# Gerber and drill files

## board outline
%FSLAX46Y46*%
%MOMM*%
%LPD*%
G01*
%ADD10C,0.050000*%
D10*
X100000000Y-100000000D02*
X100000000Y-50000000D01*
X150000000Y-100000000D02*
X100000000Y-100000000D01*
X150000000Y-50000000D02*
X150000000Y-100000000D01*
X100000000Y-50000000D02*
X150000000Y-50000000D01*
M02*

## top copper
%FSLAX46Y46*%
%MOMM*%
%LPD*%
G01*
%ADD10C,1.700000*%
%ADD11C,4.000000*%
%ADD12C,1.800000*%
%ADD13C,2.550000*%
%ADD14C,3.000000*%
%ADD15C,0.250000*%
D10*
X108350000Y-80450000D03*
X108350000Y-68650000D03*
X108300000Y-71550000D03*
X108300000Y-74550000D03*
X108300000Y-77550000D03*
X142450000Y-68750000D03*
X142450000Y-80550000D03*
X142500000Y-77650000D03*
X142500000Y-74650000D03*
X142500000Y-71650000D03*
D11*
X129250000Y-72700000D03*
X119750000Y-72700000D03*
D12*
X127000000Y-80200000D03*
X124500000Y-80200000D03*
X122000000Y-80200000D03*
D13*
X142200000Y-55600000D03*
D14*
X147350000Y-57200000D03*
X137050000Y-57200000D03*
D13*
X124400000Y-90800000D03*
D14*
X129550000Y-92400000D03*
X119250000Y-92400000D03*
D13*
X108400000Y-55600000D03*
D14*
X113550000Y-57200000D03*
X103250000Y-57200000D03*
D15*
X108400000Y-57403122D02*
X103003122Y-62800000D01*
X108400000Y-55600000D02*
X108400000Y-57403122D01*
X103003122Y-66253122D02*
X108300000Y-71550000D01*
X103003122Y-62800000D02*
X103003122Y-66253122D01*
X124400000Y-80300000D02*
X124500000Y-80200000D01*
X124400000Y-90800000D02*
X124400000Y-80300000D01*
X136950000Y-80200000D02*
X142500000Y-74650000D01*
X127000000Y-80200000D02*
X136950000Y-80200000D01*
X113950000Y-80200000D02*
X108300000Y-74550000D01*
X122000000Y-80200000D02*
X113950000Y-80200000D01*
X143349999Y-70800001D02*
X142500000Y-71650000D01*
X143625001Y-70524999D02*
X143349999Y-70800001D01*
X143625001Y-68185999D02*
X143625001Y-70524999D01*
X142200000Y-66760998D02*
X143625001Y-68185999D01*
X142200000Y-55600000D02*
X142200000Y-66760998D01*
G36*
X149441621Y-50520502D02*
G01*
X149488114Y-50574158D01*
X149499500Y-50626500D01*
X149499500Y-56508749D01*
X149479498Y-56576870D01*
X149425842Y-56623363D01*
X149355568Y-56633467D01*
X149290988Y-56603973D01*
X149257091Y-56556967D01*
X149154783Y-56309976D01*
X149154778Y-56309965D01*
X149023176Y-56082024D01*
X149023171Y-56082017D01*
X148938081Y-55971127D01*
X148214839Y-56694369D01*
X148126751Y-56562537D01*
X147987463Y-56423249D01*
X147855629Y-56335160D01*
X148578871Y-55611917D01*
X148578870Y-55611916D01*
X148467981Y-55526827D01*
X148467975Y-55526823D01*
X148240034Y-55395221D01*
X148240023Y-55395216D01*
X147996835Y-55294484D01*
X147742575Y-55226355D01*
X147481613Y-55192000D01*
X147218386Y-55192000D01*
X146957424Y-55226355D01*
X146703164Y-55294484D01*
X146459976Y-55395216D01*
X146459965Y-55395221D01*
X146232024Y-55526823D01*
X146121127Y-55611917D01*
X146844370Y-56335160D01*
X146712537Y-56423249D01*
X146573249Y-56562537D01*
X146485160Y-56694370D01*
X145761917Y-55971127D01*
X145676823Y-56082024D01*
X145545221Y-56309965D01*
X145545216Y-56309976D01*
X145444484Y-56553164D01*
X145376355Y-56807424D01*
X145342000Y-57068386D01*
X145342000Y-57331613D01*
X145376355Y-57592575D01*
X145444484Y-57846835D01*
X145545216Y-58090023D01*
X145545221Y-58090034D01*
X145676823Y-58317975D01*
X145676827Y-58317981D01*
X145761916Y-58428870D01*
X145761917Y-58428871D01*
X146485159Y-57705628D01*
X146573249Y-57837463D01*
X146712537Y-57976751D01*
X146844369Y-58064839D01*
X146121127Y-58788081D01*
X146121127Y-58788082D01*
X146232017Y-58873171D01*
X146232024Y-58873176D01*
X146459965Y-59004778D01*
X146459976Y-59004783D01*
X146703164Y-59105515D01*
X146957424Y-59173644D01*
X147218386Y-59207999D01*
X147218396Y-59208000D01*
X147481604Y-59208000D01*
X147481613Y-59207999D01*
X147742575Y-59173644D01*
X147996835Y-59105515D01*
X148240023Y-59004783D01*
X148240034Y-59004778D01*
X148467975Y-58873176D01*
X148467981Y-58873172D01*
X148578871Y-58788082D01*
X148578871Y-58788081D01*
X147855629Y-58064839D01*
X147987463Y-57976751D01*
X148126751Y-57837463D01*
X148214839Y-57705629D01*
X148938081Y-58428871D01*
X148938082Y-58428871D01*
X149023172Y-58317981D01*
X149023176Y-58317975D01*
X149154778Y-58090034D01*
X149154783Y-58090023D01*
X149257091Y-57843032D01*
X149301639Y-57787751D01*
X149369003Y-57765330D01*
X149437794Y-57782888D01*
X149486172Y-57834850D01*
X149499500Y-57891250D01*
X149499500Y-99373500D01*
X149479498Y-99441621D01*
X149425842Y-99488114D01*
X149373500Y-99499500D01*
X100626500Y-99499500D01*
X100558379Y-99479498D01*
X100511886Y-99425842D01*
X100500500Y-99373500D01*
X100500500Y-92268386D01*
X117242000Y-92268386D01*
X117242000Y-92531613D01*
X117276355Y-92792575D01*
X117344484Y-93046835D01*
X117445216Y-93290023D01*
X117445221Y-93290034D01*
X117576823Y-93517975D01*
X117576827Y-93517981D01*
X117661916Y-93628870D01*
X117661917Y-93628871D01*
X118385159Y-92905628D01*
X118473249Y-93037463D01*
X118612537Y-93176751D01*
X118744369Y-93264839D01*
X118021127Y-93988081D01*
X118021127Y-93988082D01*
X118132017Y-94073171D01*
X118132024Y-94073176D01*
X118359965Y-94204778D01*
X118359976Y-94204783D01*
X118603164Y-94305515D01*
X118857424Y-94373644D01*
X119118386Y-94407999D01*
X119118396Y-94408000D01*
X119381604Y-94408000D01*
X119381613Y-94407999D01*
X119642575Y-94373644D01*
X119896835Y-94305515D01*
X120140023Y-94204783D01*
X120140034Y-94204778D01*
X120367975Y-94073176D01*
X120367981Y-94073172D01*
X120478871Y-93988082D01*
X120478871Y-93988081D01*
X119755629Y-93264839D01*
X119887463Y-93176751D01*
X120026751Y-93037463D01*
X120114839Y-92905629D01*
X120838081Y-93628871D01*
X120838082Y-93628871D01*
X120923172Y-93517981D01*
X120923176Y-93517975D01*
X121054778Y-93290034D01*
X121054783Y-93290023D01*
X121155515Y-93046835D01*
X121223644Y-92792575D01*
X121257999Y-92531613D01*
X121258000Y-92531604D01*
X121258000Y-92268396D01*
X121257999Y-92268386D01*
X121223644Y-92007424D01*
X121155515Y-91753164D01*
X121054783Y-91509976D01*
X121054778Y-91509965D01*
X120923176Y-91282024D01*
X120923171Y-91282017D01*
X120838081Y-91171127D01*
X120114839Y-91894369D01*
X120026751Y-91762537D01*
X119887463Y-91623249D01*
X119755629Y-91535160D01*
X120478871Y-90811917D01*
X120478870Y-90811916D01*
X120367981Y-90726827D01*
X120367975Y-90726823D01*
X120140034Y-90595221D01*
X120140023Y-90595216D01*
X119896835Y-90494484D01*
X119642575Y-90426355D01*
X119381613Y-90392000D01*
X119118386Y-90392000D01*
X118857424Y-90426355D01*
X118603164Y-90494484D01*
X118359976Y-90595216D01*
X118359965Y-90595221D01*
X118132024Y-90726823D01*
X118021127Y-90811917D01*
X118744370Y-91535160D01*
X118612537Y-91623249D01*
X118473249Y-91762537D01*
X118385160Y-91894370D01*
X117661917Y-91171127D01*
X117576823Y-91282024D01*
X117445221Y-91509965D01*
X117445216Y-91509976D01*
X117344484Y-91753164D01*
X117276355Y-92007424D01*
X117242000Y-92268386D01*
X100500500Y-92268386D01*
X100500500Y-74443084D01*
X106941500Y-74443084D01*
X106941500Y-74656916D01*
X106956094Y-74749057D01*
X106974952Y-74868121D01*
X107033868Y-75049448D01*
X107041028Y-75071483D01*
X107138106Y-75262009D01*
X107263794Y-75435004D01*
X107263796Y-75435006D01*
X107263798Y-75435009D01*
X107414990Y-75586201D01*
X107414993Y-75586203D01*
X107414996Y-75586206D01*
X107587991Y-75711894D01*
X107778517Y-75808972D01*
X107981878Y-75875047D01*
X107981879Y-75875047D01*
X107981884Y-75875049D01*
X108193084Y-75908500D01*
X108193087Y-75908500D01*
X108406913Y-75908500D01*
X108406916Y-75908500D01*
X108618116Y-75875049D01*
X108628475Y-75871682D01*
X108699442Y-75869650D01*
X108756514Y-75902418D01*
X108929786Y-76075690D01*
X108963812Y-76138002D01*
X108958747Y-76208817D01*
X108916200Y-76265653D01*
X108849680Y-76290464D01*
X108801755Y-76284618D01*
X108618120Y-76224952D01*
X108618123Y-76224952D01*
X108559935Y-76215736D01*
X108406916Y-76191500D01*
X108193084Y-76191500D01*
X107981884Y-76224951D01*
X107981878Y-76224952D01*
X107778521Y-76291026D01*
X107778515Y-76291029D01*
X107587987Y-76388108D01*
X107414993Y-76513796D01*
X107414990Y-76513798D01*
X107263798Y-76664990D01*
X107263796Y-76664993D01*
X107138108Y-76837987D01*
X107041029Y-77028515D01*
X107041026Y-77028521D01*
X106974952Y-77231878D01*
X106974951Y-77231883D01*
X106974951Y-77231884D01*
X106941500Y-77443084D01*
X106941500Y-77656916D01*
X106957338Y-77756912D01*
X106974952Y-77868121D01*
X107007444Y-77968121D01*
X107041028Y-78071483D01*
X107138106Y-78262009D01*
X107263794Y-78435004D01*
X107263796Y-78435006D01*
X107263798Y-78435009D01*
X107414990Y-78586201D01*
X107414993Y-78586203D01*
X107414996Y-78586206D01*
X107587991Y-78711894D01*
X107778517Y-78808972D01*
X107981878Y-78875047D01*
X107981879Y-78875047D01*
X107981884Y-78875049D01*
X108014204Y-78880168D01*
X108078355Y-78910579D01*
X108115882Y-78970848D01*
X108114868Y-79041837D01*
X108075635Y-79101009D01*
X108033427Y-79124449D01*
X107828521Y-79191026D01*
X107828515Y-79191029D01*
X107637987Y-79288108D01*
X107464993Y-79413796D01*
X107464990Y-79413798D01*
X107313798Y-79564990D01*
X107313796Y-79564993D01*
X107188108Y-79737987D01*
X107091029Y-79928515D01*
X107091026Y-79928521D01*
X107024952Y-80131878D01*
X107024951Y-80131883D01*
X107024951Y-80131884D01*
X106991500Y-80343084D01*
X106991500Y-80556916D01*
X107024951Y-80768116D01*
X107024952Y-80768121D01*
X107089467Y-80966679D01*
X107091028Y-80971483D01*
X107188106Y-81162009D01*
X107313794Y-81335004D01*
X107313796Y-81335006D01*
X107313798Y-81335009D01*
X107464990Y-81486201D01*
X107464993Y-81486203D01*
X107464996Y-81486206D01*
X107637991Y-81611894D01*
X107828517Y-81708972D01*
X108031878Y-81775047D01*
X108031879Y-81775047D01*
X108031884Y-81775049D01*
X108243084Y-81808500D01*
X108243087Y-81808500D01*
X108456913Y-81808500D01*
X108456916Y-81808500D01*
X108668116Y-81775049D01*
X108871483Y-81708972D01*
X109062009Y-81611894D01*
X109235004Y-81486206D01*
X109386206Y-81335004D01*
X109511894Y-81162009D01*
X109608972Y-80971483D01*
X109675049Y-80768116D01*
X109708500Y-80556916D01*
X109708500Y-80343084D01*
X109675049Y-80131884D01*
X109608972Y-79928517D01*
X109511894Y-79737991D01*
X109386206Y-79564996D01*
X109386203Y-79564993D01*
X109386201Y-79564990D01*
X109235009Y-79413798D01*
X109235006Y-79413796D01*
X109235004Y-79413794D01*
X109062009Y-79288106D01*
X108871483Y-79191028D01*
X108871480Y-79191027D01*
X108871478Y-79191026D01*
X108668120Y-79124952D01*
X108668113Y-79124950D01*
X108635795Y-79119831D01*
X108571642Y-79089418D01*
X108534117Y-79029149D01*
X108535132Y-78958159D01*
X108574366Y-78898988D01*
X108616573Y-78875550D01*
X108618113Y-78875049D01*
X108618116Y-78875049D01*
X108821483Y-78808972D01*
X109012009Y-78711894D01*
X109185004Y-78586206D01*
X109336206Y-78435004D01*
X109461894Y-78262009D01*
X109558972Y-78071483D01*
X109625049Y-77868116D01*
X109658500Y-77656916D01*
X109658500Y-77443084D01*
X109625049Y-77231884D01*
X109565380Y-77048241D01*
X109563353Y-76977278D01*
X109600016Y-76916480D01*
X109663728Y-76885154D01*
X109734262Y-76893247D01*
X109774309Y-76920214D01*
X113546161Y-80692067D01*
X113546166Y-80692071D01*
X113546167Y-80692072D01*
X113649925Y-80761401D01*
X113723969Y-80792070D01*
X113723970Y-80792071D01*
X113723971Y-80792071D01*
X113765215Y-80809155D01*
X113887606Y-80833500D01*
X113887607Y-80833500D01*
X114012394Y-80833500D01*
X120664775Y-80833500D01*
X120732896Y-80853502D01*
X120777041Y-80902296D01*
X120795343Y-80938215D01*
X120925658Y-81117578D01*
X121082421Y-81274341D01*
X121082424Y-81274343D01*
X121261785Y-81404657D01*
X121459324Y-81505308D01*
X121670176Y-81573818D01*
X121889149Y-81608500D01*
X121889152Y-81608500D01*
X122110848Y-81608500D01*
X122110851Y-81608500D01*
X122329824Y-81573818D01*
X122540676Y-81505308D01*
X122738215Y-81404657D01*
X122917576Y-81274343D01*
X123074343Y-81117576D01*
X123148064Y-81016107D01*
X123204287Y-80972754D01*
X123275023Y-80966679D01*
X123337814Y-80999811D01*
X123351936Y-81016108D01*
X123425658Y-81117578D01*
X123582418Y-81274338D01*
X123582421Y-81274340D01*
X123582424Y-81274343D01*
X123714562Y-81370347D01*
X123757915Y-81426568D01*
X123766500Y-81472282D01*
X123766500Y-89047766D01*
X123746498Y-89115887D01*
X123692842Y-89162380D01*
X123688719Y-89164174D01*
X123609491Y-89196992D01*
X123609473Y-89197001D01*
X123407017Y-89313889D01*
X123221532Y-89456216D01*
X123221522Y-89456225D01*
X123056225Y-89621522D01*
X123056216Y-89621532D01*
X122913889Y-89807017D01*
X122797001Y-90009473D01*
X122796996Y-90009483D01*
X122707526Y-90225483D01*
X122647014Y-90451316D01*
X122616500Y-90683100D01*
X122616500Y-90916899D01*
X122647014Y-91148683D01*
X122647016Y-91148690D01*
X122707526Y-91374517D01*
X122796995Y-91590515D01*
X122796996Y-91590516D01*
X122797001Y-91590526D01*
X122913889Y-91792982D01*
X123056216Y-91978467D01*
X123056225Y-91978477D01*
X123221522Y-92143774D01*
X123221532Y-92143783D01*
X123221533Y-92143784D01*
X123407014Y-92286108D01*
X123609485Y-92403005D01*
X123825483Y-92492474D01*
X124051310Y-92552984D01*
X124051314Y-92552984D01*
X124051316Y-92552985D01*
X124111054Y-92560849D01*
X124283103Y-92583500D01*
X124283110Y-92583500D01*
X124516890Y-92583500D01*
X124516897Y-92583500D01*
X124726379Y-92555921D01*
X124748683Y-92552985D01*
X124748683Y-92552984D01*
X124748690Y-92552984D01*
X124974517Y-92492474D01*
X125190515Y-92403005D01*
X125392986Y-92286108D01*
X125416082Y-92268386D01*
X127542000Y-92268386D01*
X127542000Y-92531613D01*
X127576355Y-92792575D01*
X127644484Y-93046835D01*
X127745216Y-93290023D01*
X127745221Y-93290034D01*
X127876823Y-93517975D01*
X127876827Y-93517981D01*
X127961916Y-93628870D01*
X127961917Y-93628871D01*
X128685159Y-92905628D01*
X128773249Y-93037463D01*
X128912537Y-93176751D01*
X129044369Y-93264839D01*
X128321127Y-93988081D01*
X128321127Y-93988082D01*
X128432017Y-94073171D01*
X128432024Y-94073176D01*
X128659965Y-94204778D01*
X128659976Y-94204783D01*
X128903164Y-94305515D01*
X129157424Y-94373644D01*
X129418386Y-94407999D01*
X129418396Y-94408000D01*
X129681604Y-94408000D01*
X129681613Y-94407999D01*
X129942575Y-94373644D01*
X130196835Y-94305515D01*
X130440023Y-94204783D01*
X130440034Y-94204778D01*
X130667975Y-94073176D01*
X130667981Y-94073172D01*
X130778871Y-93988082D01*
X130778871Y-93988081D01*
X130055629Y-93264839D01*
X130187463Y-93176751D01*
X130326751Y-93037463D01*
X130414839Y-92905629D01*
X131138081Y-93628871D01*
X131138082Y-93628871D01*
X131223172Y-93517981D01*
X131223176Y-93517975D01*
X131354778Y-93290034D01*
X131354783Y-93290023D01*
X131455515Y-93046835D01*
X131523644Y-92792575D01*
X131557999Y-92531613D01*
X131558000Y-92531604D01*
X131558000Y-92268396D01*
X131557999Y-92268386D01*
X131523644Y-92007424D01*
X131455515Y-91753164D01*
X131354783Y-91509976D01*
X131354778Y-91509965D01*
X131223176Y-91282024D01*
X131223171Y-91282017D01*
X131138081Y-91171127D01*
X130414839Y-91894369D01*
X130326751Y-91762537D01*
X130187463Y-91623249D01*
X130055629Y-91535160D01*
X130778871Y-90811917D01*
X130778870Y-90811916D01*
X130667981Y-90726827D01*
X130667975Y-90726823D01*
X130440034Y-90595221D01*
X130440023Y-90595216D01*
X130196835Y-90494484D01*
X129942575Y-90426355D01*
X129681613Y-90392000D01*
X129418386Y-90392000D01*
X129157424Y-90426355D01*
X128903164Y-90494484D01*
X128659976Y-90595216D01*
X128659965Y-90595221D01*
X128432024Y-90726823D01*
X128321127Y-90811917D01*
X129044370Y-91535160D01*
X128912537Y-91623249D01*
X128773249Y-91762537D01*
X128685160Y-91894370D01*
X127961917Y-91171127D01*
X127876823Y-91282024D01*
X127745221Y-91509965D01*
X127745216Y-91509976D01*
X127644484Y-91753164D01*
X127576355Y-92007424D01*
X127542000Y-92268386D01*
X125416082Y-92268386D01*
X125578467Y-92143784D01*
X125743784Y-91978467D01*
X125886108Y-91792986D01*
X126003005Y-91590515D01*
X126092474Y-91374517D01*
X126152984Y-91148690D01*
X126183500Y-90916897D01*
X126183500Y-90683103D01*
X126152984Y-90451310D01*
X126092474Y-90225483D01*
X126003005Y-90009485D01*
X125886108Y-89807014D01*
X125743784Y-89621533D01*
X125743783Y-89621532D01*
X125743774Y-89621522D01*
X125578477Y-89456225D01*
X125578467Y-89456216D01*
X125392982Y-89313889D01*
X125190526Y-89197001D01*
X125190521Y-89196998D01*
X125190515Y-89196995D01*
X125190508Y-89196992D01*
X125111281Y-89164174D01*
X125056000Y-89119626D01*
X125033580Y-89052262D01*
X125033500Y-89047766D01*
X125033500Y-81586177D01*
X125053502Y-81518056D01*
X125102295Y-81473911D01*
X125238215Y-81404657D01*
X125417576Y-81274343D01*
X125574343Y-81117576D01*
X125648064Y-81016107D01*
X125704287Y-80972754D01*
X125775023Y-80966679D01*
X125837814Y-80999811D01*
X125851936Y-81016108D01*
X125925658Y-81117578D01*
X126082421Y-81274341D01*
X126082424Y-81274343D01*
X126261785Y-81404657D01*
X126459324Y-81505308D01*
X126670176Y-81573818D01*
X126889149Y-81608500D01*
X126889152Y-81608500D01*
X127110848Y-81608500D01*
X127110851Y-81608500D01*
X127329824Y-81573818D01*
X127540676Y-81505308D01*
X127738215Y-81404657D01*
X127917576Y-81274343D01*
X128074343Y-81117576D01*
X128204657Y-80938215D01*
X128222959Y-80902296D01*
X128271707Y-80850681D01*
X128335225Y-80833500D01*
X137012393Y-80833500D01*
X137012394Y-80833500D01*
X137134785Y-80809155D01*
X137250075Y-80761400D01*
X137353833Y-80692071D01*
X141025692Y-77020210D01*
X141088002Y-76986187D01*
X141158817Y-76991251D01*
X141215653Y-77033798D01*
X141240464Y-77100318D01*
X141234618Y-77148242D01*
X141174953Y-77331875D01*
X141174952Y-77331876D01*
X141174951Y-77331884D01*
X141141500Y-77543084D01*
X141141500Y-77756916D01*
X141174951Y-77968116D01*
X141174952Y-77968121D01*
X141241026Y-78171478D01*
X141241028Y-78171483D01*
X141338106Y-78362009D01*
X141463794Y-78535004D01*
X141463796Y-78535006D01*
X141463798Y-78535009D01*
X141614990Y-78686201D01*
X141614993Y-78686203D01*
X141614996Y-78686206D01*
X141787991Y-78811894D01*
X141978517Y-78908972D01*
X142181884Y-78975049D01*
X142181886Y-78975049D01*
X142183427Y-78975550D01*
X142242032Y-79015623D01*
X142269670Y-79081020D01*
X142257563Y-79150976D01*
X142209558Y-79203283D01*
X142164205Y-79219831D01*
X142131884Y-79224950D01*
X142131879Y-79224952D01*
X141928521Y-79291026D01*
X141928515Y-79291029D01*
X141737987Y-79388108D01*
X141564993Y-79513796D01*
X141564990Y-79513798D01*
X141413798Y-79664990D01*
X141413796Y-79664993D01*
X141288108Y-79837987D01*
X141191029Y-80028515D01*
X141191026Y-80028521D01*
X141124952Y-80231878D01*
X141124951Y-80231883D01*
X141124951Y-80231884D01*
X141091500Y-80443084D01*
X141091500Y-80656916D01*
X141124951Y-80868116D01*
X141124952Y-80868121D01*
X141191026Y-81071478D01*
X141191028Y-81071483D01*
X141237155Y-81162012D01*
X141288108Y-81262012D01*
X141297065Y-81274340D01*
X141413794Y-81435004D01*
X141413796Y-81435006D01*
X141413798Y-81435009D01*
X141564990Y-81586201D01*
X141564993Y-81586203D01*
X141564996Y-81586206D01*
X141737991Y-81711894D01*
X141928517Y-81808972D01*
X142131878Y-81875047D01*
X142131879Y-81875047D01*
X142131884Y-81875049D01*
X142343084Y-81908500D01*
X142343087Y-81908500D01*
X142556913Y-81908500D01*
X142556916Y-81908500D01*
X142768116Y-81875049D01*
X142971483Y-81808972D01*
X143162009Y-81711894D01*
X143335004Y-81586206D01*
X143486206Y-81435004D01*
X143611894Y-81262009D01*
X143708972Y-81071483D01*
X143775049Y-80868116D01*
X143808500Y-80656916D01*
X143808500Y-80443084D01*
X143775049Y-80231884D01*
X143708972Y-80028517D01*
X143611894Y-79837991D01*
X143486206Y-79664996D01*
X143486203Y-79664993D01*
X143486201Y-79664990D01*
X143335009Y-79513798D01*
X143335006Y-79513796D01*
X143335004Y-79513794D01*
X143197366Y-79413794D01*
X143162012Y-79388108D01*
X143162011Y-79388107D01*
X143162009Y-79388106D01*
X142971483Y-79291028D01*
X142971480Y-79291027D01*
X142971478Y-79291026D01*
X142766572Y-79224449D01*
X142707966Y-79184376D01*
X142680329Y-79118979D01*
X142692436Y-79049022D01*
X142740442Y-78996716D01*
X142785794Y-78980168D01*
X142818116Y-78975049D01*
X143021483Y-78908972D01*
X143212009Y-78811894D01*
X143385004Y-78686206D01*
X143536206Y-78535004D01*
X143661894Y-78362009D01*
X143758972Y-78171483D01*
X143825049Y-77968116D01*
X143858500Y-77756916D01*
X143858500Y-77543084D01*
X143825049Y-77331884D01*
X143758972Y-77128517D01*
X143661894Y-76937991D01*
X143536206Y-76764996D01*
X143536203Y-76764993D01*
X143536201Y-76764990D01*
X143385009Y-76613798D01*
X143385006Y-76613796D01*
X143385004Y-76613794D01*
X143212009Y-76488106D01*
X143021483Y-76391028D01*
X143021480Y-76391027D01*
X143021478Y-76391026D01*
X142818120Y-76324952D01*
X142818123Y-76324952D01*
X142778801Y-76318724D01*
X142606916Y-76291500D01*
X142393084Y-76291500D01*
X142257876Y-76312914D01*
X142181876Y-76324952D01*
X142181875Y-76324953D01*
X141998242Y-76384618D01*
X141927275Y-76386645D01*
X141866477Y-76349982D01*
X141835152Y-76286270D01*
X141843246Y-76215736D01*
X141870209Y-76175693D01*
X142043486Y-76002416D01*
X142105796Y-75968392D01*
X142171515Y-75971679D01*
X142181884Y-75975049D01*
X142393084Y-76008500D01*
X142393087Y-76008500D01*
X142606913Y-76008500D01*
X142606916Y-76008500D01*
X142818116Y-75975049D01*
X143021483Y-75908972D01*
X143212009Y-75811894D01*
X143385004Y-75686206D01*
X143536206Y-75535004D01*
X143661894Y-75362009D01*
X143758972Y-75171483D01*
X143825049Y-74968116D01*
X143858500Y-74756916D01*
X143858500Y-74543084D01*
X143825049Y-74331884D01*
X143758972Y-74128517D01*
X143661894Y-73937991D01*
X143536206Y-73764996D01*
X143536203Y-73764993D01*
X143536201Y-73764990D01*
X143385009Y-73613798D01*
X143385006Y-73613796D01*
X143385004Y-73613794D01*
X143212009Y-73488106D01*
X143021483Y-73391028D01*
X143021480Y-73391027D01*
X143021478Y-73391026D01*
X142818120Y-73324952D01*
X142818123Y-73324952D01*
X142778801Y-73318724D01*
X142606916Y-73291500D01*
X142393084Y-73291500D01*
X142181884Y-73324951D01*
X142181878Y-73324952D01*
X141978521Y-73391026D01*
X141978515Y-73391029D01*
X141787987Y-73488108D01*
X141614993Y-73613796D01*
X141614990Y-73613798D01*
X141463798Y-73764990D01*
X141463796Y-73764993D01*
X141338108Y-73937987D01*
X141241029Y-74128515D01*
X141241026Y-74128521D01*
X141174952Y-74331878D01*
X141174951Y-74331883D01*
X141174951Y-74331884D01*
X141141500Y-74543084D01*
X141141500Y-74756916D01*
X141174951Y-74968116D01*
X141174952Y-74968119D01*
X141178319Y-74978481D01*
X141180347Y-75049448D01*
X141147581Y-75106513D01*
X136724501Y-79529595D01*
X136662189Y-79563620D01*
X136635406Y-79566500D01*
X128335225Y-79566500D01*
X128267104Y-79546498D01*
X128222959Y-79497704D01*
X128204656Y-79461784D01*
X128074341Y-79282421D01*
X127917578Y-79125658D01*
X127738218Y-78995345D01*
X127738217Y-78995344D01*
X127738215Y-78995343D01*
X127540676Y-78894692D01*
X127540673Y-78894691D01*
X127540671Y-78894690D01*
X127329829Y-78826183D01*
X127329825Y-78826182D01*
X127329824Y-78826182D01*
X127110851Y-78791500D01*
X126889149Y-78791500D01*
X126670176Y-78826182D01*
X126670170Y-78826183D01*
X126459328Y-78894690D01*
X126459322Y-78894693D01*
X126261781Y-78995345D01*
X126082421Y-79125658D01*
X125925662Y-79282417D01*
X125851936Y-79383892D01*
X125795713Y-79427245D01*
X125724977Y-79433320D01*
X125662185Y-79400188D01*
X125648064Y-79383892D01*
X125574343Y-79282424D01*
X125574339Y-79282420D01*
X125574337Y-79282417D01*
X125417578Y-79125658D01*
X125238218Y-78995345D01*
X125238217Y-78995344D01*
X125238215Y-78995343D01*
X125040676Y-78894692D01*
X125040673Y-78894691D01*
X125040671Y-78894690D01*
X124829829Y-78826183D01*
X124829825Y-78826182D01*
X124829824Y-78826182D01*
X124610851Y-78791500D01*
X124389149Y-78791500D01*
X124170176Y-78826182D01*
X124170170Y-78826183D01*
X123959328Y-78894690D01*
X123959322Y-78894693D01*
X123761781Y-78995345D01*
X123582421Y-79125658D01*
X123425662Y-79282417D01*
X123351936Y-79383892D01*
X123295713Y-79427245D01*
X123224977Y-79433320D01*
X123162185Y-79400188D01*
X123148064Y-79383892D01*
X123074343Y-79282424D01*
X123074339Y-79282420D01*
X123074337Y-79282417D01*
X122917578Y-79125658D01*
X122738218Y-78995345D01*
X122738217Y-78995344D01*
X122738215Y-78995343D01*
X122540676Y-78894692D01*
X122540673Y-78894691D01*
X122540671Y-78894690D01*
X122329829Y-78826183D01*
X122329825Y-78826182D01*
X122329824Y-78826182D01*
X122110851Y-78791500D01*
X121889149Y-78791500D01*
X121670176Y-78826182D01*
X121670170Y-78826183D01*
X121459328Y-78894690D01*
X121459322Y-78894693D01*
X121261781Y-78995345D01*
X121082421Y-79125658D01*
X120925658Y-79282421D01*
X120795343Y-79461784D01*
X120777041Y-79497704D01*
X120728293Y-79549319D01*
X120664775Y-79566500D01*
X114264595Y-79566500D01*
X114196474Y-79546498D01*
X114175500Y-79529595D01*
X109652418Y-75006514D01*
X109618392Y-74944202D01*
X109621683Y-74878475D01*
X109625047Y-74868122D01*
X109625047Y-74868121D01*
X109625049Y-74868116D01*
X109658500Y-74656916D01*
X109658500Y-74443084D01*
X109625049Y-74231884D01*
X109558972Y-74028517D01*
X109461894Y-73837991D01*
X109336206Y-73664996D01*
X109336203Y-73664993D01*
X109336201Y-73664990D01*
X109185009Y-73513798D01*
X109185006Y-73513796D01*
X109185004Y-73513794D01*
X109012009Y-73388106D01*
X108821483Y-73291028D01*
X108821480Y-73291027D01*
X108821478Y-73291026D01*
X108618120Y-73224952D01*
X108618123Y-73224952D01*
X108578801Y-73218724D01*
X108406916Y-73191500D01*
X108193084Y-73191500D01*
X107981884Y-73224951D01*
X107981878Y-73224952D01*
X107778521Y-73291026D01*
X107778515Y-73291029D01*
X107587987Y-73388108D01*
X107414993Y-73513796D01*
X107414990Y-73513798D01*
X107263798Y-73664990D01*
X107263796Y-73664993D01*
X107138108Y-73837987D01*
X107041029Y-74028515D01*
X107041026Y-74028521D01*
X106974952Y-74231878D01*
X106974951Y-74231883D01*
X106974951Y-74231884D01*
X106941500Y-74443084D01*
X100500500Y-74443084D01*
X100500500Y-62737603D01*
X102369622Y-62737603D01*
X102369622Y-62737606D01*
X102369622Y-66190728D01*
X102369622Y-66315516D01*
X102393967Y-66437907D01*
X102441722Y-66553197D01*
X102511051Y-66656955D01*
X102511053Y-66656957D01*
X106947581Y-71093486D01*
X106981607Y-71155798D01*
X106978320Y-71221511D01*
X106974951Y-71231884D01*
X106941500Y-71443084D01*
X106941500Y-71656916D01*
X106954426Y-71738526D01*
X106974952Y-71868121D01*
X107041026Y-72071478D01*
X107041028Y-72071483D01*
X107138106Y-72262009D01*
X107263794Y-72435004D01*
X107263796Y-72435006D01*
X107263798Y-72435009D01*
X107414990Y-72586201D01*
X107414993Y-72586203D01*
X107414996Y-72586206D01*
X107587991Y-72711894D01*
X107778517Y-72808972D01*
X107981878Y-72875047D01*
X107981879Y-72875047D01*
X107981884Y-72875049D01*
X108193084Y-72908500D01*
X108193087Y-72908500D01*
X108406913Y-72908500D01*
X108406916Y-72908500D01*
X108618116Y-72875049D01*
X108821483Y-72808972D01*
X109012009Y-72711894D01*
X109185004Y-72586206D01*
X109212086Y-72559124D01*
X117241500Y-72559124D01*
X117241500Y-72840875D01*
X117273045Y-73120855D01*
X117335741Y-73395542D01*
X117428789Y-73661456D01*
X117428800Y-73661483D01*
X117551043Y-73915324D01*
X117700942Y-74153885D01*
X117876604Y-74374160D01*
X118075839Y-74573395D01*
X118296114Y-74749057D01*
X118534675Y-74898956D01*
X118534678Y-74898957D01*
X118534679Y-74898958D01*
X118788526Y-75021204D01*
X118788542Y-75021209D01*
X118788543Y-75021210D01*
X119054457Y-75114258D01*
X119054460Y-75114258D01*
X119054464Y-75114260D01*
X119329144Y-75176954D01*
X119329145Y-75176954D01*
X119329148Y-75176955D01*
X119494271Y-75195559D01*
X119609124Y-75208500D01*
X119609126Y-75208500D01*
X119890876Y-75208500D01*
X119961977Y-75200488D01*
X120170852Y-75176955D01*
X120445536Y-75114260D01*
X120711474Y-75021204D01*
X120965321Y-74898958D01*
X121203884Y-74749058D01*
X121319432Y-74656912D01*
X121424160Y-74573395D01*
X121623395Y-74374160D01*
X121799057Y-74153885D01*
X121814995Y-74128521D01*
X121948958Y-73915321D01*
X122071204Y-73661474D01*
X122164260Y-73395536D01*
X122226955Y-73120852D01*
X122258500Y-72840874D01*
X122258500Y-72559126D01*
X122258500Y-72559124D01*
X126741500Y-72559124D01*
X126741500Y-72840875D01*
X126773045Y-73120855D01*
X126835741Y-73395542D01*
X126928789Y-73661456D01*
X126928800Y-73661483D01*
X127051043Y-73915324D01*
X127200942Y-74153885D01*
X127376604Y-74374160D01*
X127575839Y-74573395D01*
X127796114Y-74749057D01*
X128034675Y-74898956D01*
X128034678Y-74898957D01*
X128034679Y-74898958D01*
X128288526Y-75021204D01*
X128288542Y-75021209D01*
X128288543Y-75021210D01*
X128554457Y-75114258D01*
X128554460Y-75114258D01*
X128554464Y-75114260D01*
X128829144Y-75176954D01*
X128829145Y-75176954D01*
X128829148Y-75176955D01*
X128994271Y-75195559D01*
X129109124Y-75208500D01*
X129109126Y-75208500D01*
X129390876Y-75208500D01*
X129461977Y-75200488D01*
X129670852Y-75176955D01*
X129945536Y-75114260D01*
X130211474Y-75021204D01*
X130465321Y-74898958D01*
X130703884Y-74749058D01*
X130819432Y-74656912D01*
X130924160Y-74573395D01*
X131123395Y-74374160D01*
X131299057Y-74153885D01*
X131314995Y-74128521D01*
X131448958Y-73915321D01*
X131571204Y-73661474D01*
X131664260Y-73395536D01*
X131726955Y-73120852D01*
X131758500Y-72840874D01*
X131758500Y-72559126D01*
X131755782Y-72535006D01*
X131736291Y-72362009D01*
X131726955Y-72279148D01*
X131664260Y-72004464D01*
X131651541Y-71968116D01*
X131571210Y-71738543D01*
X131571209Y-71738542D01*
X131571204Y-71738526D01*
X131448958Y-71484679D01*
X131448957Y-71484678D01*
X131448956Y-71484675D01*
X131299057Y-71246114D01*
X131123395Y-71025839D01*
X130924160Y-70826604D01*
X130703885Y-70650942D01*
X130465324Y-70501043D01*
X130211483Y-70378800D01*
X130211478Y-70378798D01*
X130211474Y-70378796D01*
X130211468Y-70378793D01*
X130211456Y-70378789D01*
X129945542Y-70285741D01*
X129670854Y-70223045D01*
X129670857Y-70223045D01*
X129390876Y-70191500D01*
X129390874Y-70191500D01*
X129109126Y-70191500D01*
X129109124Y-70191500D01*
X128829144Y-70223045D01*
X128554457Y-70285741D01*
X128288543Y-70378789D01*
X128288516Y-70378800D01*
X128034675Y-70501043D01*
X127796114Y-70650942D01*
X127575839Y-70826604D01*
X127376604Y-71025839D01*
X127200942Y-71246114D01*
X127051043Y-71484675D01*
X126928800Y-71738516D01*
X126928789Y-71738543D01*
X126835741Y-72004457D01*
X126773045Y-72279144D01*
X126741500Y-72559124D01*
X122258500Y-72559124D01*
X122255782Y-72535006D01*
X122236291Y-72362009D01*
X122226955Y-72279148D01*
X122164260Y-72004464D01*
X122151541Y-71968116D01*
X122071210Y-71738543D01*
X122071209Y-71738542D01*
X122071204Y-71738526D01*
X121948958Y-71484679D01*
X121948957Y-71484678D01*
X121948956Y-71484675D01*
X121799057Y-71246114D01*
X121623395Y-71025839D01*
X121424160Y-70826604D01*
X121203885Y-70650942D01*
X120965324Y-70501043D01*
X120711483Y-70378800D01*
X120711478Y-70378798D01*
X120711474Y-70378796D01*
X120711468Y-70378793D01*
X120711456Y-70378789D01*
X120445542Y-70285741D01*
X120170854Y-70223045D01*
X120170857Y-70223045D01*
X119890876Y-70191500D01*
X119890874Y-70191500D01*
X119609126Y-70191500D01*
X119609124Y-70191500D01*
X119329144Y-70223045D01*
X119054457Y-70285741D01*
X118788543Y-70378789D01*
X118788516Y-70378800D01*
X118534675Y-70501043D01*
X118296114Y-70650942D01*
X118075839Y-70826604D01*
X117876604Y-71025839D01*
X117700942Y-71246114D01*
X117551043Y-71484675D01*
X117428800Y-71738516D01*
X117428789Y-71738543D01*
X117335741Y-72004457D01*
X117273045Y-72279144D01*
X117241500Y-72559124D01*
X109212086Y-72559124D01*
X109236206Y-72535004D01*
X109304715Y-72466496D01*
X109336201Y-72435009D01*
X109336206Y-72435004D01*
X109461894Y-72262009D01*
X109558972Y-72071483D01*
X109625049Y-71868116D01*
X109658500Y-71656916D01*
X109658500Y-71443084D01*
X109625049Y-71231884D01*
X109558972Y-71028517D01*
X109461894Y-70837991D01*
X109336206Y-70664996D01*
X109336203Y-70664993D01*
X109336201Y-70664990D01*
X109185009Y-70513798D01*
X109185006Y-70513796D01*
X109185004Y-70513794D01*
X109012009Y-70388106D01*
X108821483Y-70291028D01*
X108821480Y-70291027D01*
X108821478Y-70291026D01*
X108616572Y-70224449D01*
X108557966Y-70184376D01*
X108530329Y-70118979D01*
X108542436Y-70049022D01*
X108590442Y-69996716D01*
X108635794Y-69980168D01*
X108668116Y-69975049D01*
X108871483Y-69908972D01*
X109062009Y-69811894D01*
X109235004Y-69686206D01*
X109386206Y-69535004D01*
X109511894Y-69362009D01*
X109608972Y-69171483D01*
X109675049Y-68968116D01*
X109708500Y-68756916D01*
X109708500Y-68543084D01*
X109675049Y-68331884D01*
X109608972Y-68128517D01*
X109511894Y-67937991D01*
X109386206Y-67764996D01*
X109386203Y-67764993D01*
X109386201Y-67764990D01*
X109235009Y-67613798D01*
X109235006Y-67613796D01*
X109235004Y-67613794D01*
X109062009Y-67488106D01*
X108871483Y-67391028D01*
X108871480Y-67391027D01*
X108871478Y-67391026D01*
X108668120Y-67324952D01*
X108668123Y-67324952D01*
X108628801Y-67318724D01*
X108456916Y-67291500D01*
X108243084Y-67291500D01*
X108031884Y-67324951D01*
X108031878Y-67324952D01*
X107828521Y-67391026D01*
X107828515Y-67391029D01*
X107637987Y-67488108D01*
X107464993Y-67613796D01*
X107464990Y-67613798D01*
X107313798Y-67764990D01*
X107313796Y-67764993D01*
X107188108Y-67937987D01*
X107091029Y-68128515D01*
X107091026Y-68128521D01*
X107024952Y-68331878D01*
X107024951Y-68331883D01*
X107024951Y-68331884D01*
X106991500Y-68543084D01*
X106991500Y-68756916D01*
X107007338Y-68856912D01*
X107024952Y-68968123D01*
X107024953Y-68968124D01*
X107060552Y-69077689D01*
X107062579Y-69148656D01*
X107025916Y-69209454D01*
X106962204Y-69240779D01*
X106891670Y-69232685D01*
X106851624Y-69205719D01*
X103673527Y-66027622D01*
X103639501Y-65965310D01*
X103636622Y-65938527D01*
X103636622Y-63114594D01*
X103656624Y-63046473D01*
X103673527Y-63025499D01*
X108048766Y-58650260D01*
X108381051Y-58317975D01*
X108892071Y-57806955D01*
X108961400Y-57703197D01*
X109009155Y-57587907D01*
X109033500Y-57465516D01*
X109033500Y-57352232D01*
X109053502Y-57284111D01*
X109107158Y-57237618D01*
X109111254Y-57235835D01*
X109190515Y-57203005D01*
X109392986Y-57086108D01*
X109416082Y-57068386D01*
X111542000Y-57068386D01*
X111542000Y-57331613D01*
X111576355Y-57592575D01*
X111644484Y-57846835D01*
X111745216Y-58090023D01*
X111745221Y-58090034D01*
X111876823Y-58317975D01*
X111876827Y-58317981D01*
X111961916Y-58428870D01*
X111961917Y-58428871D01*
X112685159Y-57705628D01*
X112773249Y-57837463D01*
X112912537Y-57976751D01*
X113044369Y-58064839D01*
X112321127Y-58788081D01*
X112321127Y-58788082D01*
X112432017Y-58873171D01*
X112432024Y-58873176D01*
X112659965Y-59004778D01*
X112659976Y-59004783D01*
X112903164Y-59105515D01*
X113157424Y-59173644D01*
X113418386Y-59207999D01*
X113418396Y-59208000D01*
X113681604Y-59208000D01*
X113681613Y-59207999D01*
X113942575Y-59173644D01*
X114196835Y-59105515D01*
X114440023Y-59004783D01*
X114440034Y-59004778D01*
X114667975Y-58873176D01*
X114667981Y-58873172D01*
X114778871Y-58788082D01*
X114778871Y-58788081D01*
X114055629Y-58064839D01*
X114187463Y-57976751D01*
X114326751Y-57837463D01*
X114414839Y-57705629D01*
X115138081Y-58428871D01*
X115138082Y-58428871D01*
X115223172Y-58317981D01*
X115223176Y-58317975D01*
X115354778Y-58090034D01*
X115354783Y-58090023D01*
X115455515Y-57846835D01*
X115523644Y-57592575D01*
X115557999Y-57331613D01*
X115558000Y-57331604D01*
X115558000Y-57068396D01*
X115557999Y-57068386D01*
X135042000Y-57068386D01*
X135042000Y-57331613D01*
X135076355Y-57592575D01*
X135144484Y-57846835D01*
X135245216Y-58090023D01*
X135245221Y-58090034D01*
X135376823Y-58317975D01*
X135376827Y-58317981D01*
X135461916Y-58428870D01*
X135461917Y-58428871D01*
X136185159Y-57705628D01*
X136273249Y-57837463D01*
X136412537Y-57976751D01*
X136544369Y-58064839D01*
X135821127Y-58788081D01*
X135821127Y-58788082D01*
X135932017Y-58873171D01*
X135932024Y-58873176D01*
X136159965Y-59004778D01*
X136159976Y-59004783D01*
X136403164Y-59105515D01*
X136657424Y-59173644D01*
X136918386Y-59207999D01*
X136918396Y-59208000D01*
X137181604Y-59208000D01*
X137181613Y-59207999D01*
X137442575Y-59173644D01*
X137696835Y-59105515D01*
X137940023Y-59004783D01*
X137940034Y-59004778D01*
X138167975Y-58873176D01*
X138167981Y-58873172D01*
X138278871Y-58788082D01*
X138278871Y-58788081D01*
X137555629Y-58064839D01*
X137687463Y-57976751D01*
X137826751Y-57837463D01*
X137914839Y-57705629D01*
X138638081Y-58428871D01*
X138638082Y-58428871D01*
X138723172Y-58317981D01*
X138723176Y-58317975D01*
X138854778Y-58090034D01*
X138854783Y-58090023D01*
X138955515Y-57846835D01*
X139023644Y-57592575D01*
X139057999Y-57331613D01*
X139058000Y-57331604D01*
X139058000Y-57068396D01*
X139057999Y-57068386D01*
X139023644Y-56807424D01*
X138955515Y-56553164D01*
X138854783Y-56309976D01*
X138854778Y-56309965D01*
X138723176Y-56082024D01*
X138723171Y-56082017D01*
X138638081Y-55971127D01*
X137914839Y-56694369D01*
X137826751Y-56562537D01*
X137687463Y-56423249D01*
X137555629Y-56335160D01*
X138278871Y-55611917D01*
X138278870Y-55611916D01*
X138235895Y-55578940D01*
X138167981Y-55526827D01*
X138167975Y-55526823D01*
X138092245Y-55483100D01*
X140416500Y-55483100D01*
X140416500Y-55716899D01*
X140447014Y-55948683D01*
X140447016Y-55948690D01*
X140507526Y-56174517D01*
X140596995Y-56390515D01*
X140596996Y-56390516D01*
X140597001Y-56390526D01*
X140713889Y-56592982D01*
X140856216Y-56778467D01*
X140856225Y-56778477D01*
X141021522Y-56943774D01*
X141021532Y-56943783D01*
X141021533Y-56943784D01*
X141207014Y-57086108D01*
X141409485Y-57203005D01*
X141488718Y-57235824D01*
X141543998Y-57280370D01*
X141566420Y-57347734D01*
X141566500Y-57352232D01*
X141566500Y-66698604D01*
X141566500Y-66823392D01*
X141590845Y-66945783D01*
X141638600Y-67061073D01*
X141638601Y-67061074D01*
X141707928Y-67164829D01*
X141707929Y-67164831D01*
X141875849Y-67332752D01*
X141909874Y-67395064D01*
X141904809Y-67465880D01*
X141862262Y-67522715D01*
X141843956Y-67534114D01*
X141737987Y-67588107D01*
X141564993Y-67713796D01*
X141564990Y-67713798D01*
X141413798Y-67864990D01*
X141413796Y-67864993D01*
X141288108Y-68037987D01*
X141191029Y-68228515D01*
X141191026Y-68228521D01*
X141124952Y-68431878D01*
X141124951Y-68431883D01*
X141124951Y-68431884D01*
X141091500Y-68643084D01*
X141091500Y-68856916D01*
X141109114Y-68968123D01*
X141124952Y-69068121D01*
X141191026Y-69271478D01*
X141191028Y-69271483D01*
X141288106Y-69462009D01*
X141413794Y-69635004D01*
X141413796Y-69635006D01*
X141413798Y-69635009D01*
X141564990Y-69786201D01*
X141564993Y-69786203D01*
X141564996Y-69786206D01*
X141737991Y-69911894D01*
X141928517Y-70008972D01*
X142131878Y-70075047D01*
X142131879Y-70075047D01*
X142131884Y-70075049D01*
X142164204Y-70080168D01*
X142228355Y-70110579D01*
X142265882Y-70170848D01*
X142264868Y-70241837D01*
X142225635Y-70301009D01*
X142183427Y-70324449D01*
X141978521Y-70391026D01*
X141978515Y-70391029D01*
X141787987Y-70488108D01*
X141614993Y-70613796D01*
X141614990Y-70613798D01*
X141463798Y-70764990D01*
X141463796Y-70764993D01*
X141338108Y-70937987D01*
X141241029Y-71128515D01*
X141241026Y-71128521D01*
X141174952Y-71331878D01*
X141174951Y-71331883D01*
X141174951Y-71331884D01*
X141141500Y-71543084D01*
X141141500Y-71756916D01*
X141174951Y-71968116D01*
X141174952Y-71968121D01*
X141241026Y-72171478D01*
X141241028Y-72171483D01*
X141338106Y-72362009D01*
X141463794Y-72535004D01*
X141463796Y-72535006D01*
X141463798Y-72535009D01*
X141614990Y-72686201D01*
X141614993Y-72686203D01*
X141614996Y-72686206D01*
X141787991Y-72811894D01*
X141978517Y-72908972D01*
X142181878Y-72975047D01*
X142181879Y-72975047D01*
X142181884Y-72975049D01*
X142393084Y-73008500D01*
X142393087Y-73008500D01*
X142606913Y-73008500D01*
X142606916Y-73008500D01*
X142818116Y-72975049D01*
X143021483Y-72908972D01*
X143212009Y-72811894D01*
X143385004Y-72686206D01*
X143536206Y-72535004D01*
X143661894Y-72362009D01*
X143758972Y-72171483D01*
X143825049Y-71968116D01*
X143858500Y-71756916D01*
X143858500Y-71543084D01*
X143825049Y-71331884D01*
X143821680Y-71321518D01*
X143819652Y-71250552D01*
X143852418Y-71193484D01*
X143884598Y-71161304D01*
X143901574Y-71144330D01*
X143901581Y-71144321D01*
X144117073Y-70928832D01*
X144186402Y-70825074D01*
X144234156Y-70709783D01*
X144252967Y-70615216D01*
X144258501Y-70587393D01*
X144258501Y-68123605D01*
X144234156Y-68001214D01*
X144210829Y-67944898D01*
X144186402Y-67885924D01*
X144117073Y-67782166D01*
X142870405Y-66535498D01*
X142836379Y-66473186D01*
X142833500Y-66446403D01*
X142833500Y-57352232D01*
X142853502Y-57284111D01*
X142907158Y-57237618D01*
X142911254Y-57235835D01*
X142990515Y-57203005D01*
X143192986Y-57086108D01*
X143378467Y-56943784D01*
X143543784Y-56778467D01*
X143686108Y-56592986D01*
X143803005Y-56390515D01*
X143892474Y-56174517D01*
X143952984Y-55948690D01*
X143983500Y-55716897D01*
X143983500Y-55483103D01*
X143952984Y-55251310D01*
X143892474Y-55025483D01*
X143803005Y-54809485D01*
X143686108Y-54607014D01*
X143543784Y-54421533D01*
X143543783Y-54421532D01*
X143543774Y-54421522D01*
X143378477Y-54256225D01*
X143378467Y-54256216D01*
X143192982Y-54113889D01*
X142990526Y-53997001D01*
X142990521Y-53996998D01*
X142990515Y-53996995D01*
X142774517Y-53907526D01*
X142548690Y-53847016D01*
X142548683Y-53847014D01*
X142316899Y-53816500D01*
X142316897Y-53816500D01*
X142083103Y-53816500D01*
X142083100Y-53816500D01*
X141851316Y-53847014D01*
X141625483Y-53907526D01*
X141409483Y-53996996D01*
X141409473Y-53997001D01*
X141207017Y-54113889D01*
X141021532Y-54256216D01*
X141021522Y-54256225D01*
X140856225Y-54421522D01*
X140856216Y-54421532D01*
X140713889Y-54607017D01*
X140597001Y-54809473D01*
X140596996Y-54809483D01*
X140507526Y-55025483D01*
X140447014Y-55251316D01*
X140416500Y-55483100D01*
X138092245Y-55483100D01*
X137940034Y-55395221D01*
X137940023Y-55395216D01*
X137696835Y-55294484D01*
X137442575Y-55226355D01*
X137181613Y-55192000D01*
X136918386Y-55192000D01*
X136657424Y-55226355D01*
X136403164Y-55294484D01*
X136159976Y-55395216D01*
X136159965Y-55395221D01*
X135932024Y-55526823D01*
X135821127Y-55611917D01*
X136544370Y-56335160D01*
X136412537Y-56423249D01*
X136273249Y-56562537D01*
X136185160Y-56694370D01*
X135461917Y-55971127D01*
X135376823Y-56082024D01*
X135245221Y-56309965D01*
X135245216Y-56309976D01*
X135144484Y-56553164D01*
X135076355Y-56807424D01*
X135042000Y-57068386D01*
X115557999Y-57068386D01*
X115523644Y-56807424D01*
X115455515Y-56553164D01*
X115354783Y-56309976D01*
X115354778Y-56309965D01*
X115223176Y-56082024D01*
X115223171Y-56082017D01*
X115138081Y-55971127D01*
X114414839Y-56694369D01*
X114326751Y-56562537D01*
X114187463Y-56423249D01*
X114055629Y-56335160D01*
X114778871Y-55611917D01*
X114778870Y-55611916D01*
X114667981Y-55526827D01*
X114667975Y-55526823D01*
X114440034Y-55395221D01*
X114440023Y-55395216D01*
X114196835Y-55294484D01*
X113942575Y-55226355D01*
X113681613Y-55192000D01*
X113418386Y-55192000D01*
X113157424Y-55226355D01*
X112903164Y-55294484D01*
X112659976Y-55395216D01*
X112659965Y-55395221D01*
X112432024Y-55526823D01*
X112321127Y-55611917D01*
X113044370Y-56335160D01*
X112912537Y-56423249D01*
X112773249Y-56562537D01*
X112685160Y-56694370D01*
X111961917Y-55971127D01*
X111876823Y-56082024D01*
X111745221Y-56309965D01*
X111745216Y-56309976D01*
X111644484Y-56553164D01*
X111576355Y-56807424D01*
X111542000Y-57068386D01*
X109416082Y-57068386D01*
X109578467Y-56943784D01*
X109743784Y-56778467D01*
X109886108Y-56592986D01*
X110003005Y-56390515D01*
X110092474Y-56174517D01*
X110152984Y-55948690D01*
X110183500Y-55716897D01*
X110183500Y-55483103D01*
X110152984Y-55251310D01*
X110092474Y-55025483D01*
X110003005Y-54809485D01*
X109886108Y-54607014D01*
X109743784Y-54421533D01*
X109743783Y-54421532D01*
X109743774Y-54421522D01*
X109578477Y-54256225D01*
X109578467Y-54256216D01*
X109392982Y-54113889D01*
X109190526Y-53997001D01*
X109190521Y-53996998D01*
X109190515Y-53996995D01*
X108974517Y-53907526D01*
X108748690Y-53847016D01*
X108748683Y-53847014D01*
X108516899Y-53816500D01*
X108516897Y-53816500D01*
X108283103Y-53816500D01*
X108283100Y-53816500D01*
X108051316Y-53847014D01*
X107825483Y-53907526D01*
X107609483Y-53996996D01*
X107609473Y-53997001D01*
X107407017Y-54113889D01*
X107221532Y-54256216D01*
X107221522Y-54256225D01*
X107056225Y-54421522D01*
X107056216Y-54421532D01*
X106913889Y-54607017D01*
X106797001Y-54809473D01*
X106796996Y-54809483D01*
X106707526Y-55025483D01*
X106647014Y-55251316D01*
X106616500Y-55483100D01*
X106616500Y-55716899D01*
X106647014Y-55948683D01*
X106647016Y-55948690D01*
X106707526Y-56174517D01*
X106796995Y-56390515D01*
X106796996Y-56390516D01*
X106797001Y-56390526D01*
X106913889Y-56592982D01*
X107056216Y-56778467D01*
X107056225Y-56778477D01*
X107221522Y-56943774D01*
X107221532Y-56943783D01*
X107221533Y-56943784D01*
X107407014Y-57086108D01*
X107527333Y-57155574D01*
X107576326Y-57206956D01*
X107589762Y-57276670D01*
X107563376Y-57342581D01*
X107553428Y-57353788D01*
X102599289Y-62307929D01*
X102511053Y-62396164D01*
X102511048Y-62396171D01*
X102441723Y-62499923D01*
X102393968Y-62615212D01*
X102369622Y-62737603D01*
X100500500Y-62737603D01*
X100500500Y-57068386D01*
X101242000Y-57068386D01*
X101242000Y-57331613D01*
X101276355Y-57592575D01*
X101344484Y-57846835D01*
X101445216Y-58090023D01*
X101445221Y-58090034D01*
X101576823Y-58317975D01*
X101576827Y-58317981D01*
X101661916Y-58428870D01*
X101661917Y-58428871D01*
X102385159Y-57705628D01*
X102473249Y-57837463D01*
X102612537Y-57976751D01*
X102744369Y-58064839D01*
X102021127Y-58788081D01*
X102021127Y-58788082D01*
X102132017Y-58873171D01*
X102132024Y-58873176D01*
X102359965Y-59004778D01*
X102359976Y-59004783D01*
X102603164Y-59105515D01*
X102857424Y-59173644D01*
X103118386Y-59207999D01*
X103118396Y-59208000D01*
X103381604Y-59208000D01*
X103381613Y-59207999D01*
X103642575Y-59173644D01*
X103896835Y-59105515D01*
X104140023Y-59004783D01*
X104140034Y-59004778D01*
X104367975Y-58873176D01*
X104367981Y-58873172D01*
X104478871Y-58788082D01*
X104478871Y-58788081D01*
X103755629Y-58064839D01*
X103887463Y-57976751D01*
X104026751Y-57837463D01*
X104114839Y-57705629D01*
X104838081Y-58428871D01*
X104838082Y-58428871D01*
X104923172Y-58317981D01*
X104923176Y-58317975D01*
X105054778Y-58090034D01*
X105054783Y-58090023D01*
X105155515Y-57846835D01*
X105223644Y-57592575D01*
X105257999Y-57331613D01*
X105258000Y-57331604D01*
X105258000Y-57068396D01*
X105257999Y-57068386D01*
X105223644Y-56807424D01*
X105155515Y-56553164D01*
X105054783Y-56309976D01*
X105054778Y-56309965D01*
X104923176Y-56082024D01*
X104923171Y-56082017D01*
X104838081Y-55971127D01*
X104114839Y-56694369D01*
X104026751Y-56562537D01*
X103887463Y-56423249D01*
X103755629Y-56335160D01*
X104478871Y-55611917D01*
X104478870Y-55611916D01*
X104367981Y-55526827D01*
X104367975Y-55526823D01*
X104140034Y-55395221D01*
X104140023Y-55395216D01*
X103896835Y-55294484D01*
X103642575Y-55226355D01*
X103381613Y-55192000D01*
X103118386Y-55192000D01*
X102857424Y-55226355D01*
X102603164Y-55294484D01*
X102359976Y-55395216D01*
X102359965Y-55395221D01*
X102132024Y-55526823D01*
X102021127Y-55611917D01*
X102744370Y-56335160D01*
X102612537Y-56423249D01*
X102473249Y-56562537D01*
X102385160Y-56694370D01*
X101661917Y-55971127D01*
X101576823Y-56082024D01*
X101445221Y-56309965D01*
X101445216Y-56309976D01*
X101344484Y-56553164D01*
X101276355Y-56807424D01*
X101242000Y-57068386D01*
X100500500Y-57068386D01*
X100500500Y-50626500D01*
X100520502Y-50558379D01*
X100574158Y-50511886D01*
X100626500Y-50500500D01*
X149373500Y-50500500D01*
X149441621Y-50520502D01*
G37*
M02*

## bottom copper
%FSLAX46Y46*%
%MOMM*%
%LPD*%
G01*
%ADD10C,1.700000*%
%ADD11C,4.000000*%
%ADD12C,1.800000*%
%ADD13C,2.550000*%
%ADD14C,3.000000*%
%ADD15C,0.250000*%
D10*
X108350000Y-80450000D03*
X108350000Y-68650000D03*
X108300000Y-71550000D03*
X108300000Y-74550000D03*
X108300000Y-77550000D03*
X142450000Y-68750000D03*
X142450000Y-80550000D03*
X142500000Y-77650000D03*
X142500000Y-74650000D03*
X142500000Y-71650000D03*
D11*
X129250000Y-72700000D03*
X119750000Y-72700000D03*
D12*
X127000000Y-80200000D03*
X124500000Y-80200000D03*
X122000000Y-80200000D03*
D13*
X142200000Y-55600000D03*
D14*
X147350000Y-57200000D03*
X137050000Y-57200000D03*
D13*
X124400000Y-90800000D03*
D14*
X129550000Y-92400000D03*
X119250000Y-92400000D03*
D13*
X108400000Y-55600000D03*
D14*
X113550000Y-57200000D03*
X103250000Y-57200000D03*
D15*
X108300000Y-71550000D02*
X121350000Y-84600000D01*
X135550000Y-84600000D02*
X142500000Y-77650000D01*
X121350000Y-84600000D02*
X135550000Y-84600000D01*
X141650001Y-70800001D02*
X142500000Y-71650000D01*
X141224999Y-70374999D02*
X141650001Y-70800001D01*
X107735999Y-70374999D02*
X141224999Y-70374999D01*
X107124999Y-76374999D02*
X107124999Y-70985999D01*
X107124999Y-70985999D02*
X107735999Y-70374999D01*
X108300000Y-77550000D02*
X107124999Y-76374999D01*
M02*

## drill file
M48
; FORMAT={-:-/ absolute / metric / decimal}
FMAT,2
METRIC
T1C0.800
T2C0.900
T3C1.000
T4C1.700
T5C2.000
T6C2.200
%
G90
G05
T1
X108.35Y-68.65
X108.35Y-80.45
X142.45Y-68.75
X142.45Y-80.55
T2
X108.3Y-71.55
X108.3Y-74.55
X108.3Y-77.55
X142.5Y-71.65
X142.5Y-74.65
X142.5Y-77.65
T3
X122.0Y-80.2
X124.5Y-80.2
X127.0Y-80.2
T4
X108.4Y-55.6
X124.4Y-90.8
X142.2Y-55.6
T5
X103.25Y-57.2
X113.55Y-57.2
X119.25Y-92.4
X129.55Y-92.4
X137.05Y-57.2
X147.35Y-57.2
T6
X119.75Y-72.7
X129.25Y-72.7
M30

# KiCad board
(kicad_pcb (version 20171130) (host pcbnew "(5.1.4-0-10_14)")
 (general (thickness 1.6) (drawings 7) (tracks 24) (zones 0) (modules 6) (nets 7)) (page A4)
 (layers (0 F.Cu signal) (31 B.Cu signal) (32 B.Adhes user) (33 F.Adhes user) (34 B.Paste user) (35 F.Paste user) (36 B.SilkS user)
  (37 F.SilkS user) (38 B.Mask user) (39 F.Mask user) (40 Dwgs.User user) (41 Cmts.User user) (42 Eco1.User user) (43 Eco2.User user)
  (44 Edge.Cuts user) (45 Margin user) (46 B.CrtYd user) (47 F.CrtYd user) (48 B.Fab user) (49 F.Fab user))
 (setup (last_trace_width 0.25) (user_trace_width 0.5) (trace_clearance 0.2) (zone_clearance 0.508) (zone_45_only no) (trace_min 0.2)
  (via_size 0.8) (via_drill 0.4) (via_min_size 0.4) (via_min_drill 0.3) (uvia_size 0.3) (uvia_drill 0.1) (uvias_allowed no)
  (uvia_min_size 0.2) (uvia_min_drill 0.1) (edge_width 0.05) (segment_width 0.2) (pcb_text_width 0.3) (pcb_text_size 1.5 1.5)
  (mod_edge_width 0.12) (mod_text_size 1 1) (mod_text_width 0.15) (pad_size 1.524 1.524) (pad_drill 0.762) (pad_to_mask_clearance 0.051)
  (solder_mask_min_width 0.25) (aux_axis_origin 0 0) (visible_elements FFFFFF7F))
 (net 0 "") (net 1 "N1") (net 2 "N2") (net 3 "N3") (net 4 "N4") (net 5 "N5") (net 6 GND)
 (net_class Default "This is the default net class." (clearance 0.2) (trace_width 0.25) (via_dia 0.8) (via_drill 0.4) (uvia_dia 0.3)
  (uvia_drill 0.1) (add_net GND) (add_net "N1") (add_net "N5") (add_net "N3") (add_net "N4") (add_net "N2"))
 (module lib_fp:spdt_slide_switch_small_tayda (layer F.Cu) (at 108.2 74.6 90)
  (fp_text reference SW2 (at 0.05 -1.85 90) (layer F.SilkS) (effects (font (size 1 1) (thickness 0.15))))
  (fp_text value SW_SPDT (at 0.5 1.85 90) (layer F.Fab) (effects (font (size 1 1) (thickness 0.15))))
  (pad "" thru_hole circle (at -5.85 0.15 90) (size 1.7 1.7) (drill 0.8) (layers *.Cu *.Mask))
  (pad "" thru_hole circle (at 5.95 0.15 90) (size 1.7 1.7) (drill 0.8) (layers *.Cu *.Mask))
  (pad 3 thru_hole circle (at 3.05 0.1 90) (size 1.7 1.7) (drill 0.9) (layers *.Cu *.Mask) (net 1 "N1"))
  (pad 2 thru_hole circle (at 0.05 0.1 90) (size 1.7 1.7) (drill 0.9) (layers *.Cu *.Mask) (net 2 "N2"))
  (pad 1 thru_hole circle (at -2.95 0.1 90) (size 1.7 1.7) (drill 0.9) (layers *.Cu *.Mask) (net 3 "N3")))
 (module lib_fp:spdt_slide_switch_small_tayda (layer F.Cu) (at 142.6 74.6 270)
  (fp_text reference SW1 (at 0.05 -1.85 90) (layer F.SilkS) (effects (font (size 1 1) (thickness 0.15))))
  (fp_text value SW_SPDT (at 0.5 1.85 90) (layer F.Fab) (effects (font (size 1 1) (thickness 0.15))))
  (pad "" thru_hole circle (at -5.85 0.15 270) (size 1.7 1.7) (drill 0.8) (layers *.Cu *.Mask))
  (pad "" thru_hole circle (at 5.95 0.15 270) (size 1.7 1.7) (drill 0.8) (layers *.Cu *.Mask))
  (pad 3 thru_hole circle (at 3.05 0.1 270) (size 1.7 1.7) (drill 0.9) (layers *.Cu *.Mask) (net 1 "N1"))
  (pad 2 thru_hole circle (at 0.05 0.1 270) (size 1.7 1.7) (drill 0.9) (layers *.Cu *.Mask) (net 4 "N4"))
  (pad 1 thru_hole circle (at -2.95 0.1 270) (size 1.7 1.7) (drill 0.9) (layers *.Cu *.Mask) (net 3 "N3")))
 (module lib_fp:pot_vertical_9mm (layer F.Cu) (at 127 80.2 90)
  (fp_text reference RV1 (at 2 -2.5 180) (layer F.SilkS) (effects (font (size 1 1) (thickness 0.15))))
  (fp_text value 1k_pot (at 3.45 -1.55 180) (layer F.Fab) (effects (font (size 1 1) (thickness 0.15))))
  (pad "" np_thru_hole circle (at 7.5 2.25 90) (size 4 4) (drill 2.2) (layers *.Cu *.Mask))
  (pad "" np_thru_hole circle (at 7.5 -7.25 90) (size 4 4) (drill 2.2) (layers *.Cu *.Mask))
  (pad 1 thru_hole circle (at 0 0 90) (size 1.8 1.8) (drill 1) (layers *.Cu *.Mask) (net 4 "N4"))
  (pad 2 thru_hole circle (at 0 -2.5 90) (size 1.8 1.8) (drill 1) (layers *.Cu *.Mask) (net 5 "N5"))
  (pad 3 thru_hole circle (at 0 -5 90) (size 1.8 1.8) (drill 1) (layers *.Cu *.Mask) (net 2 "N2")))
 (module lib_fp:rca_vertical (layer F.Cu) (at 142.2 57.2)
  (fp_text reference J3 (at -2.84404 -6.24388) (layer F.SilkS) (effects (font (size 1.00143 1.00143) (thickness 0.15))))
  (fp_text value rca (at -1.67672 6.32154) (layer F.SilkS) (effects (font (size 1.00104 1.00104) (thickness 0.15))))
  (pad 1 thru_hole circle (at 0 -1.6) (size 2.55 2.55) (drill 1.7) (layers *.Cu *.Mask) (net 3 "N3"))
  (pad 2 thru_hole circle (at 5.15 0) (size 3 3) (drill 2) (layers *.Cu *.Mask) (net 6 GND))
  (pad 2 thru_hole circle (at -5.15 0) (size 3 3) (drill 2) (layers *.Cu *.Mask) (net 6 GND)))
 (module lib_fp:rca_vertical (layer F.Cu) (at 124.4 92.4)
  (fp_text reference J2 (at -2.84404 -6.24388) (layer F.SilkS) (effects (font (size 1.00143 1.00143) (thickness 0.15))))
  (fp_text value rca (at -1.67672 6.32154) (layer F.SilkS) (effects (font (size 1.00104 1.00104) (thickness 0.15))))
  (pad 1 thru_hole circle (at 0 -1.6) (size 2.55 2.55) (drill 1.7) (layers *.Cu *.Mask) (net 5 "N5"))
  (pad 2 thru_hole circle (at 5.15 0) (size 3 3) (drill 2) (layers *.Cu *.Mask) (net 6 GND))
  (pad 2 thru_hole circle (at -5.15 0) (size 3 3) (drill 2) (layers *.Cu *.Mask) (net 6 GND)))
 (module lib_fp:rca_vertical (layer F.Cu) (at 108.4 57.2)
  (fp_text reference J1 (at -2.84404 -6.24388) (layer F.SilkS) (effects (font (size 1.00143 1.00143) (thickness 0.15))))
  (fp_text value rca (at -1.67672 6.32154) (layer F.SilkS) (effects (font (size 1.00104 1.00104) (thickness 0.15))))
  (pad 1 thru_hole circle (at 0 -1.6) (size 2.55 2.55) (drill 1.7) (layers *.Cu *.Mask) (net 1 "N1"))
  (pad 2 thru_hole circle (at 5.15 0) (size 3 3) (drill 2) (layers *.Cu *.Mask) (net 6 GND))
  (pad 2 thru_hole circle (at -5.15 0) (size 3 3) (drill 2) (layers *.Cu *.Mask) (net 6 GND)))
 (gr_line (start 100 100) (end 100 50) (layer Edge.Cuts) (width 0.05))
 (gr_line (start 150 100) (end 100 100) (layer Edge.Cuts) (width 0.05))
 (gr_line (start 150 50) (end 150 100) (layer Edge.Cuts) (width 0.05))
 (gr_line (start 100 50) (end 150 50) (layer Edge.Cuts) (width 0.05))
 (segment (start 108.4 57.403122) (end 103.003122 62.8) (width 0.25) (layer F.Cu) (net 1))
 (segment (start 108.4 55.6) (end 108.4 57.403122) (width 0.25) (layer F.Cu) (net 1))
 (segment (start 103.003122 66.253122) (end 108.3 71.55) (width 0.25) (layer F.Cu) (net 1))
 (segment (start 103.003122 62.8) (end 103.003122 66.253122) (width 0.25) (layer F.Cu) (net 1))
 (segment (start 108.3 71.55) (end 121.35 84.6) (width 0.25) (layer B.Cu) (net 1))
 (segment (start 135.55 84.6) (end 142.5 77.65) (width 0.25) (layer B.Cu) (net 1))
 (segment (start 121.35 84.6) (end 135.55 84.6) (width 0.25) (layer B.Cu) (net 1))
 (segment (start 124.4 80.3) (end 124.5 80.2) (width 0.25) (layer F.Cu) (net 5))
 (segment (start 124.4 90.8) (end 124.4 80.3) (width 0.25) (layer F.Cu) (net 5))
 (segment (start 136.95 80.2) (end 142.5 74.65) (width 0.25) (layer F.Cu) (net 4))
 (segment (start 127 80.2) (end 136.95 80.2) (width 0.25) (layer F.Cu) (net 4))
 (segment (start 113.95 80.2) (end 108.3 74.55) (width 0.25) (layer F.Cu) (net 2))
 (segment (start 122 80.2) (end 113.95 80.2) (width 0.25) (layer F.Cu) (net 2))
 (segment (start 143.349999 70.800001) (end 142.5 71.65) (width 0.25) (layer F.Cu) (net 3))
 (segment (start 143.625001 70.524999) (end 143.349999 70.800001) (width 0.25) (layer F.Cu) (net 3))
 (segment (start 143.625001 68.185999) (end 143.625001 70.524999) (width 0.25) (layer F.Cu) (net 3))
 (segment (start 142.2 66.760998) (end 143.625001 68.185999) (width 0.25) (layer F.Cu) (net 3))
 (segment (start 142.2 55.6) (end 142.2 66.760998) (width 0.25) (layer F.Cu) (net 3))
 (segment (start 141.650001 70.800001) (end 142.5 71.65) (width 0.25) (layer B.Cu) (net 3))
 (segment (start 141.224999 70.374999) (end 141.650001 70.800001) (width 0.25) (layer B.Cu) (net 3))
 (segment (start 107.735999 70.374999) (end 141.224999 70.374999) (width 0.25) (layer B.Cu) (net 3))
 (segment (start 107.124999 76.374999) (end 107.124999 70.985999) (width 0.25) (layer B.Cu) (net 3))
 (segment (start 107.124999 70.985999) (end 107.735999 70.374999) (width 0.25) (layer B.Cu) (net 3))
 (segment (start 108.3 77.55) (end 107.124999 76.374999) (width 0.25) (layer B.Cu) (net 3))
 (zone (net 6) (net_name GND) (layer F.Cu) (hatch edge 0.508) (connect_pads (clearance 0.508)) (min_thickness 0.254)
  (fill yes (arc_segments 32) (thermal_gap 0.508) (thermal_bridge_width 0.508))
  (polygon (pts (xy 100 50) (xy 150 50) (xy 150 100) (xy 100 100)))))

